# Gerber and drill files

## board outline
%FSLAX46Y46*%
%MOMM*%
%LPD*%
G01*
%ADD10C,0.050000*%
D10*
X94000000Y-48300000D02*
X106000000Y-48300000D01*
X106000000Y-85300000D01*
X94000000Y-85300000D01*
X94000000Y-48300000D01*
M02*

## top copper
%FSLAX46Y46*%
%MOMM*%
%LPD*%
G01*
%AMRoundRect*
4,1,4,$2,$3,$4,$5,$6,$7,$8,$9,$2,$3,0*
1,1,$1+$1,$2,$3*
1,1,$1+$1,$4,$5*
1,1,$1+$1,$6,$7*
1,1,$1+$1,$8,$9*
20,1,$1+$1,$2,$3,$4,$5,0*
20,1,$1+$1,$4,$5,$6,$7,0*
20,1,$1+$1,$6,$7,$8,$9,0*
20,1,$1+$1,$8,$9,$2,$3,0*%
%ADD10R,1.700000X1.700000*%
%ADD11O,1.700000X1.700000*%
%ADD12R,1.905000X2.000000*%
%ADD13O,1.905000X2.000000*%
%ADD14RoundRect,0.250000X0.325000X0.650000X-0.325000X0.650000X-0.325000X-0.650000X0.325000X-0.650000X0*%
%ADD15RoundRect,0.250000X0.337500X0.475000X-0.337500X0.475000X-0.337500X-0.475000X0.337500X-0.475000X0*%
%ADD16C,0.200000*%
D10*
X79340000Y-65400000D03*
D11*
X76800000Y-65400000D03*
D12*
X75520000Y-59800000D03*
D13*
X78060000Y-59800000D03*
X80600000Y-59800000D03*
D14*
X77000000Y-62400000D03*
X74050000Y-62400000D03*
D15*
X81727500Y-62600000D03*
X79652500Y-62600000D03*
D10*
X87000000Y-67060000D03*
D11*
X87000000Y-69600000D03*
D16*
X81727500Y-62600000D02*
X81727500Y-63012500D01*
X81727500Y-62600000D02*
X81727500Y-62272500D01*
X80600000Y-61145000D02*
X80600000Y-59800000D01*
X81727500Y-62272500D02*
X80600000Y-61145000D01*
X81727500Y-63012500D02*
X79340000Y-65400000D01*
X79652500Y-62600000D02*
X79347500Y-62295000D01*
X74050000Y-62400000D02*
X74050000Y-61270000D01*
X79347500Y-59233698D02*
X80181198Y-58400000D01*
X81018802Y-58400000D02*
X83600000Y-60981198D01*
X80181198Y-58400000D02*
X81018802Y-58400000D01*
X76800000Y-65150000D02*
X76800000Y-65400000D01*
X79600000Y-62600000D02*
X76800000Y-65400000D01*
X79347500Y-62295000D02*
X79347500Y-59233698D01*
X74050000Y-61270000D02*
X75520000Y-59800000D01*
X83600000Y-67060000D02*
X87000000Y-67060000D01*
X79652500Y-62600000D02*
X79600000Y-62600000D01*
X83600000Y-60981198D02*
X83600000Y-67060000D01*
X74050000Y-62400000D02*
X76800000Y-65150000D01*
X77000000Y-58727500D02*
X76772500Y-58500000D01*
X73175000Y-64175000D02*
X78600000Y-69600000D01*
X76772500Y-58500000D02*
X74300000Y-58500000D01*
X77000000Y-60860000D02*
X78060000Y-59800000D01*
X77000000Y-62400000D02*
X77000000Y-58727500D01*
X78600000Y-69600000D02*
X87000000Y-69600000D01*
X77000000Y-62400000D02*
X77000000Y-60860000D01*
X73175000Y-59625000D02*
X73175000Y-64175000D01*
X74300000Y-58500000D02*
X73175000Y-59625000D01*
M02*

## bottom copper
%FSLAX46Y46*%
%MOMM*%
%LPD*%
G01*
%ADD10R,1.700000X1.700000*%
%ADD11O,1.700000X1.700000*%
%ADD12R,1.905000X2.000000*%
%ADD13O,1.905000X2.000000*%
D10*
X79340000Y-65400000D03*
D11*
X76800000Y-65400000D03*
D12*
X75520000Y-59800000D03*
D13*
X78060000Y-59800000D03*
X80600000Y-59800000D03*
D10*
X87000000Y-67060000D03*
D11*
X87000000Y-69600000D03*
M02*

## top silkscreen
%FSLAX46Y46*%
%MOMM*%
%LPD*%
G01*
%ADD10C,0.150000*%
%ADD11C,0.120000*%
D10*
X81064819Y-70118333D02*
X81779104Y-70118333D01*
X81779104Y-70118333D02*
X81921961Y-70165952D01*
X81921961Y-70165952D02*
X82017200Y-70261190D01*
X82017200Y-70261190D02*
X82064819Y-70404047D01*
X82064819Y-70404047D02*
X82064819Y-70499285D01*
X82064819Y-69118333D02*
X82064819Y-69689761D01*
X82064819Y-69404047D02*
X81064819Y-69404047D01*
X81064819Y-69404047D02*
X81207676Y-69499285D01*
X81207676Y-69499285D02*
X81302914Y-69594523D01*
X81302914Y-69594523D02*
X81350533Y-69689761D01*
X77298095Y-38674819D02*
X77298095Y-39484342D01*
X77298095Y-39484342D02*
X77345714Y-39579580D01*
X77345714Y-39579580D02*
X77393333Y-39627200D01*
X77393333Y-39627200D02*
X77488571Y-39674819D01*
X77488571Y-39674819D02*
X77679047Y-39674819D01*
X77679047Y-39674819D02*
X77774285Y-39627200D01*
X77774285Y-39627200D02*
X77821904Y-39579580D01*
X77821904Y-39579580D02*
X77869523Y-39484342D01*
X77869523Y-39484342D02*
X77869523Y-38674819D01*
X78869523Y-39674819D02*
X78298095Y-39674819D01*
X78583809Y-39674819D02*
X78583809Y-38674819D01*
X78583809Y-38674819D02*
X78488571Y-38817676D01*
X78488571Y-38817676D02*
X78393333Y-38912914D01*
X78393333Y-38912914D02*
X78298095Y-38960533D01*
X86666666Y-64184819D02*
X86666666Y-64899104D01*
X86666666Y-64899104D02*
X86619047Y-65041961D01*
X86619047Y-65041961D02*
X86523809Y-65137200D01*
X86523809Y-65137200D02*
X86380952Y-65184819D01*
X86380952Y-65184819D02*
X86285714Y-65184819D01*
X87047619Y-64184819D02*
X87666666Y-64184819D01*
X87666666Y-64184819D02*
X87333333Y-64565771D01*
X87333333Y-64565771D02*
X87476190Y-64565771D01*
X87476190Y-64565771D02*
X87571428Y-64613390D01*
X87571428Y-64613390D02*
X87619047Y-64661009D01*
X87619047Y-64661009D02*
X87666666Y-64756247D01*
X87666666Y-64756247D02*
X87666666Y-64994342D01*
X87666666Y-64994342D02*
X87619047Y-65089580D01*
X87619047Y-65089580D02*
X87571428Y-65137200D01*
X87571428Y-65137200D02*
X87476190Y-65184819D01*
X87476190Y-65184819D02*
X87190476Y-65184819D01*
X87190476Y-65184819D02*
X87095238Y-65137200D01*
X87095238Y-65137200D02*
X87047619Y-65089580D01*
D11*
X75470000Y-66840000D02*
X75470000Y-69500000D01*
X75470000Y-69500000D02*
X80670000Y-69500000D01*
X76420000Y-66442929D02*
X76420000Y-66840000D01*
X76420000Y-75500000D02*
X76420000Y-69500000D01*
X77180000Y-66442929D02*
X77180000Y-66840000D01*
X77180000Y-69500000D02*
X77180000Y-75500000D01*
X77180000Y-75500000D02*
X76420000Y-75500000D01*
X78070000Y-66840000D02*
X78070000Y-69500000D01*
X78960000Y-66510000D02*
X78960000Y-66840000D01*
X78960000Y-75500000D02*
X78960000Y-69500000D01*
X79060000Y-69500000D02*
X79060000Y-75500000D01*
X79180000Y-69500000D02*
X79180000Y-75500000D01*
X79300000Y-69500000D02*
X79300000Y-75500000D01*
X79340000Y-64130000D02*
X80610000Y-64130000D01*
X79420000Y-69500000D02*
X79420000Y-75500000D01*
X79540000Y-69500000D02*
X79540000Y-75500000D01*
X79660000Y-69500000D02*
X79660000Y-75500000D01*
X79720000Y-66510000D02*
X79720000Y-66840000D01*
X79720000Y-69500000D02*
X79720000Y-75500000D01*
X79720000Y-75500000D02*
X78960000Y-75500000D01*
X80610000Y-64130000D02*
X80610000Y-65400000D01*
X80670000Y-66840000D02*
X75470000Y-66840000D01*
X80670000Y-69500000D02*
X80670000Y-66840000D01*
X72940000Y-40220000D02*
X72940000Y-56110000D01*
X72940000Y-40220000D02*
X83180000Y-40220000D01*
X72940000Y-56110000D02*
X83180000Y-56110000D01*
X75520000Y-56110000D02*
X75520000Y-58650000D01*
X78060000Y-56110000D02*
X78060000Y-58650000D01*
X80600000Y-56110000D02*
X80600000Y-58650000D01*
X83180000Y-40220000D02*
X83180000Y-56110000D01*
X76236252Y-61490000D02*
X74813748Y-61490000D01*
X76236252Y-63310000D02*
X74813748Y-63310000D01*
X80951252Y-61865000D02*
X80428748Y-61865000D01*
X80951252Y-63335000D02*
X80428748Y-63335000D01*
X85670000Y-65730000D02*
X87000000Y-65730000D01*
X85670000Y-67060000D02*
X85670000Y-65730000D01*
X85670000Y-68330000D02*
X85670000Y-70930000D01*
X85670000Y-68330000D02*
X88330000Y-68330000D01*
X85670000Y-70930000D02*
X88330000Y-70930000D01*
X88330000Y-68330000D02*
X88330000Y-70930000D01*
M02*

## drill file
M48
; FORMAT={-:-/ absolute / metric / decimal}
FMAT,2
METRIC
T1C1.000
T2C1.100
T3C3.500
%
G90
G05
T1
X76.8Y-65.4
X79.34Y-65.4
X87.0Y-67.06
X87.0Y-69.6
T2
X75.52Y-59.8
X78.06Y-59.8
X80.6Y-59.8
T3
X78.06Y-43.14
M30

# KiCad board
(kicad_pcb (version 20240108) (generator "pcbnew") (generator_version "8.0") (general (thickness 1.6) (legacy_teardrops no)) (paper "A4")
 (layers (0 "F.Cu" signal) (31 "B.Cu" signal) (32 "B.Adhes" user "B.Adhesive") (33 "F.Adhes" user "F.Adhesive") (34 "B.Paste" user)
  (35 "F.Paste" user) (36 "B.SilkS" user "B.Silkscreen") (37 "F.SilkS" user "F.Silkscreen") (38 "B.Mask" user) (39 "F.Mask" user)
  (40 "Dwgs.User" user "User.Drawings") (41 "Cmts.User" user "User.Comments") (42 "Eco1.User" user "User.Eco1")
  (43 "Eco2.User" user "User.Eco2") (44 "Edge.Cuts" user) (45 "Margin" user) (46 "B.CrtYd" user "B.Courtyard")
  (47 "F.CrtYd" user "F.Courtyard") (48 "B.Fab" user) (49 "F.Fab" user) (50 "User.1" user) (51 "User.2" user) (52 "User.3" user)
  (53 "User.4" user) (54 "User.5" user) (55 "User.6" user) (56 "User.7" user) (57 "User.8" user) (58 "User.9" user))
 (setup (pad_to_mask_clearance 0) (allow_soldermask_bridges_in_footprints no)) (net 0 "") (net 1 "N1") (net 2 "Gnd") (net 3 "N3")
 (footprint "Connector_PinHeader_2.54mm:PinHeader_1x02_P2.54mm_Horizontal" (layer "F.Cu") (at 79.34 65.4 -90)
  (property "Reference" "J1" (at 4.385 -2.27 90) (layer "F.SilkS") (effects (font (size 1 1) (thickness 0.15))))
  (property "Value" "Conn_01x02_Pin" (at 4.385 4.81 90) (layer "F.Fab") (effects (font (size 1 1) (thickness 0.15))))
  (fp_line (start 1.44 3.87) (end 4.1 3.87) (stroke (width 0.12) (type solid)) (layer "F.SilkS"))
  (fp_line (start 4.1 3.87) (end 4.1 -1.33) (stroke (width 0.12) (type solid)) (layer "F.SilkS"))
  (fp_line (start 1.042929 2.92) (end 1.44 2.92) (stroke (width 0.12) (type solid)) (layer "F.SilkS"))
  (fp_line (start 10.1 2.92) (end 4.1 2.92) (stroke (width 0.12) (type solid)) (layer "F.SilkS"))
  (fp_line (start 1.042929 2.16) (end 1.44 2.16) (stroke (width 0.12) (type solid)) (layer "F.SilkS"))
  (fp_line (start 4.1 2.16) (end 10.1 2.16) (stroke (width 0.12) (type solid)) (layer "F.SilkS"))
  (fp_line (start 10.1 2.16) (end 10.1 2.92) (stroke (width 0.12) (type solid)) (layer "F.SilkS"))
  (fp_line (start 1.44 1.27) (end 4.1 1.27) (stroke (width 0.12) (type solid)) (layer "F.SilkS"))
  (fp_line (start 1.11 0.38) (end 1.44 0.38) (stroke (width 0.12) (type solid)) (layer "F.SilkS"))
  (fp_line (start 10.1 0.38) (end 4.1 0.38) (stroke (width 0.12) (type solid)) (layer "F.SilkS"))
  (fp_line (start 4.1 0.28) (end 10.1 0.28) (stroke (width 0.12) (type solid)) (layer "F.SilkS"))
  (fp_line (start 4.1 0.16) (end 10.1 0.16) (stroke (width 0.12) (type solid)) (layer "F.SilkS"))
  (fp_line (start 4.1 0.04) (end 10.1 0.04) (stroke (width 0.12) (type solid)) (layer "F.SilkS"))
  (fp_line (start -1.27 0) (end -1.27 -1.27) (stroke (width 0.12) (type solid)) (layer "F.SilkS"))
  (fp_line (start 4.1 -0.08) (end 10.1 -0.08) (stroke (width 0.12) (type solid)) (layer "F.SilkS"))
  (fp_line (start 4.1 -0.2) (end 10.1 -0.2) (stroke (width 0.12) (type solid)) (layer "F.SilkS"))
  (fp_line (start 4.1 -0.32) (end 10.1 -0.32) (stroke (width 0.12) (type solid)) (layer "F.SilkS"))
  (fp_line (start 1.11 -0.38) (end 1.44 -0.38) (stroke (width 0.12) (type solid)) (layer "F.SilkS"))
  (fp_line (start 4.1 -0.38) (end 10.1 -0.38) (stroke (width 0.12) (type solid)) (layer "F.SilkS"))
  (fp_line (start 10.1 -0.38) (end 10.1 0.38) (stroke (width 0.12) (type solid)) (layer "F.SilkS"))
  (fp_line (start -1.27 -1.27) (end 0 -1.27) (stroke (width 0.12) (type solid)) (layer "F.SilkS"))
  (fp_line (start 1.44 -1.33) (end 1.44 3.87) (stroke (width 0.12) (type solid)) (layer "F.SilkS"))
  (fp_line (start 4.1 -1.33) (end 1.44 -1.33) (stroke (width 0.12) (type solid)) (layer "F.SilkS"))
  (pad "1" thru_hole rect (at 0 0 270) (size 1.7 1.7) (drill 1) (layers "*.Cu" "*.Mask") (remove_unused_layers no) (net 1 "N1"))
  (pad "2" thru_hole oval (at 0 2.54 270) (size 1.7 1.7) (drill 1) (layers "*.Cu" "*.Mask") (remove_unused_layers no) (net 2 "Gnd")))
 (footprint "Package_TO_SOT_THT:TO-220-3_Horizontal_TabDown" (layer "F.Cu") (at 75.52 59.8)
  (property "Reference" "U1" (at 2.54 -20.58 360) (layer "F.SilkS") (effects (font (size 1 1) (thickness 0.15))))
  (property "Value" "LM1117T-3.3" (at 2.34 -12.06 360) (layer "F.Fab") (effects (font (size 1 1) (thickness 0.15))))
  (fp_line (start -2.58 -19.58) (end -2.58 -3.69) (stroke (width 0.12) (type solid)) (layer "F.SilkS"))
  (fp_line (start -2.58 -19.58) (end 7.66 -19.58) (stroke (width 0.12) (type solid)) (layer "F.SilkS"))
  (fp_line (start -2.58 -3.69) (end 7.66 -3.69) (stroke (width 0.12) (type solid)) (layer "F.SilkS"))
  (fp_line (start 0 -3.69) (end 0 -1.15) (stroke (width 0.12) (type solid)) (layer "F.SilkS"))
  (fp_line (start 2.54 -3.69) (end 2.54 -1.15) (stroke (width 0.12) (type solid)) (layer "F.SilkS"))
  (fp_line (start 5.08 -3.69) (end 5.08 -1.15) (stroke (width 0.12) (type solid)) (layer "F.SilkS"))
  (fp_line (start 7.66 -19.58) (end 7.66 -3.69) (stroke (width 0.12) (type solid)) (layer "F.SilkS"))
  (pad "" np_thru_hole circle (at 2.54 -16.66) (size 3.5 3.5) (drill 3.5) (layers "*.Cu" "*.Mask"))
  (pad "1" thru_hole rect (at 0 0) (size 1.905 2) (drill 1.1) (layers "*.Cu" "*.Mask") (remove_unused_layers no) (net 2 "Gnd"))
  (pad "2" thru_hole oval (at 2.54 0) (size 1.905 2) (drill 1.1) (layers "*.Cu" "*.Mask") (remove_unused_layers no) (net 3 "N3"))
  (pad "3" thru_hole oval (at 5.08 0) (size 1.905 2) (drill 1.1) (layers "*.Cu" "*.Mask") (remove_unused_layers no) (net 1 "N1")))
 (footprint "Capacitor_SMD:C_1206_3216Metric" (layer "F.Cu") (at 75.525 62.4 180)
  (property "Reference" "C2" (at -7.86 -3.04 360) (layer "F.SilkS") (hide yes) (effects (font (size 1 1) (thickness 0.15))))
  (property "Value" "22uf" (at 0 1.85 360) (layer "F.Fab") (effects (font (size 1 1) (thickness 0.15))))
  (fp_line (start -0.711252 0.91) (end 0.711252 0.91) (stroke (width 0.12) (type solid)) (layer "F.SilkS"))
  (fp_line (start -0.711252 -0.91) (end 0.711252 -0.91) (stroke (width 0.12) (type solid)) (layer "F.SilkS"))
  (pad "1" smd roundrect (at -1.475 0 180) (size 1.15 1.8) (layers "F.Cu" "F.Paste" "F.Mask") (roundrect_rratio 0.217391) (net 3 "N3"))
  (pad "2" smd roundrect (at 1.475 0 180) (size 1.15 1.8) (layers "F.Cu" "F.Paste" "F.Mask") (roundrect_rratio 0.217391) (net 2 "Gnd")))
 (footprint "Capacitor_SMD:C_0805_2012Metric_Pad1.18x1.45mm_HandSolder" (layer "F.Cu") (at 80.69 62.6 180)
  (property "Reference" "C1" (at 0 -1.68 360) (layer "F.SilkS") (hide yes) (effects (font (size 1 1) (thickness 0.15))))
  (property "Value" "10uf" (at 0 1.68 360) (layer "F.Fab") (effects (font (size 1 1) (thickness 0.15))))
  (fp_line (start -0.261252 0.735) (end 0.261252 0.735) (stroke (width 0.12) (type solid)) (layer "F.SilkS"))
  (fp_line (start -0.261252 -0.735) (end 0.261252 -0.735) (stroke (width 0.12) (type solid)) (layer "F.SilkS"))
  (pad "1" smd roundrect (at -1.0375 0 180) (size 1.175 1.45) (layers "F.Cu" "F.Paste" "F.Mask") (roundrect_rratio 0.212766) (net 1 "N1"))
  (pad "2" smd roundrect (at 1.0375 0 180) (size 1.175 1.45) (layers "F.Cu" "F.Paste" "F.Mask") (roundrect_rratio 0.212766) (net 2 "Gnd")))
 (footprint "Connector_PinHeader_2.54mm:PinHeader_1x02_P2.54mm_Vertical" (layer "F.Cu") (at 87 67.06)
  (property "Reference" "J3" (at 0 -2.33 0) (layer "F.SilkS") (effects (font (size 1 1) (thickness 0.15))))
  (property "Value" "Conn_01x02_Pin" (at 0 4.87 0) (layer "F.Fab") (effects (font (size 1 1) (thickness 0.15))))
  (fp_line (start -1.33 -1.33) (end 0 -1.33) (stroke (width 0.12) (type solid)) (layer "F.SilkS"))
  (fp_line (start -1.33 0) (end -1.33 -1.33) (stroke (width 0.12) (type solid)) (layer "F.SilkS"))
  (fp_line (start -1.33 1.27) (end -1.33 3.87) (stroke (width 0.12) (type solid)) (layer "F.SilkS"))
  (fp_line (start -1.33 1.27) (end 1.33 1.27) (stroke (width 0.12) (type solid)) (layer "F.SilkS"))
  (fp_line (start -1.33 3.87) (end 1.33 3.87) (stroke (width 0.12) (type solid)) (layer "F.SilkS"))
  (fp_line (start 1.33 1.27) (end 1.33 3.87) (stroke (width 0.12) (type solid)) (layer "F.SilkS"))
  (pad "1" thru_hole rect (at 0 0) (size 1.7 1.7) (drill 1) (layers "*.Cu" "*.Mask") (remove_unused_layers no) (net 2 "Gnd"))
  (pad "2" thru_hole oval (at 0 2.54) (size 1.7 1.7) (drill 1) (layers "*.Cu" "*.Mask") (remove_unused_layers no) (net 3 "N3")))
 (gr_rect (start 94 48.3) (end 106 85.3) (stroke (width 0.05) (type default)) (fill none) (layer "Edge.Cuts"))
 (segment (start 81.7275 62.6) (end 81.7275 63.0125) (width 0.2) (layer "F.Cu") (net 1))
 (segment (start 81.7275 62.6) (end 81.7275 62.2725) (width 0.2) (layer "F.Cu") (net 1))
 (segment (start 80.6 61.145) (end 80.6 59.8) (width 0.2) (layer "F.Cu") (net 1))
 (segment (start 81.7275 62.2725) (end 80.6 61.145) (width 0.2) (layer "F.Cu") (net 1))
 (segment (start 81.7275 63.0125) (end 79.34 65.4) (width 0.2) (layer "F.Cu") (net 1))
 (segment (start 79.6525 62.6) (end 79.3475 62.295) (width 0.2) (layer "F.Cu") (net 2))
 (segment (start 74.05 62.4) (end 74.05 61.27) (width 0.2) (layer "F.Cu") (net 2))
 (segment (start 79.3475 59.233698) (end 80.181198 58.4) (width 0.2) (layer "F.Cu") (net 2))
 (segment (start 81.018802 58.4) (end 83.6 60.981198) (width 0.2) (layer "F.Cu") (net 2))
 (segment (start 80.181198 58.4) (end 81.018802 58.4) (width 0.2) (layer "F.Cu") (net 2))
 (segment (start 76.8 65.15) (end 76.8 65.4) (width 0.2) (layer "F.Cu") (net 2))
 (segment (start 79.6 62.6) (end 76.8 65.4) (width 0.2) (layer "F.Cu") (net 2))
 (segment (start 79.3475 62.295) (end 79.3475 59.233698) (width 0.2) (layer "F.Cu") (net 2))
 (segment (start 74.05 61.27) (end 75.52 59.8) (width 0.2) (layer "F.Cu") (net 2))
 (segment (start 83.6 67.06) (end 87 67.06) (width 0.2) (layer "F.Cu") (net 2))
 (segment (start 79.6525 62.6) (end 79.6 62.6) (width 0.2) (layer "F.Cu") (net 2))
 (segment (start 83.6 60.981198) (end 83.6 67.06) (width 0.2) (layer "F.Cu") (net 2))
 (segment (start 74.05 62.4) (end 76.8 65.15) (width 0.2) (layer "F.Cu") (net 2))
 (segment (start 77 58.7275) (end 76.7725 58.5) (width 0.2) (layer "F.Cu") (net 3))
 (segment (start 73.175 64.175) (end 78.6 69.6) (width 0.2) (layer "F.Cu") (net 3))
 (segment (start 76.7725 58.5) (end 74.3 58.5) (width 0.2) (layer "F.Cu") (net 3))
 (segment (start 77 60.86) (end 78.06 59.8) (width 0.2) (layer "F.Cu") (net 3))
 (segment (start 77 62.4) (end 77 58.7275) (width 0.2) (layer "F.Cu") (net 3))
 (segment (start 78.6 69.6) (end 87 69.6) (width 0.2) (layer "F.Cu") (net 3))
 (segment (start 77 62.4) (end 77 60.86) (width 0.2) (layer "F.Cu") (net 3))
 (segment (start 73.175 59.625) (end 73.175 64.175) (width 0.2) (layer "F.Cu") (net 3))
 (segment (start 74.3 58.5) (end 73.175 59.625) (width 0.2) (layer "F.Cu") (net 3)))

